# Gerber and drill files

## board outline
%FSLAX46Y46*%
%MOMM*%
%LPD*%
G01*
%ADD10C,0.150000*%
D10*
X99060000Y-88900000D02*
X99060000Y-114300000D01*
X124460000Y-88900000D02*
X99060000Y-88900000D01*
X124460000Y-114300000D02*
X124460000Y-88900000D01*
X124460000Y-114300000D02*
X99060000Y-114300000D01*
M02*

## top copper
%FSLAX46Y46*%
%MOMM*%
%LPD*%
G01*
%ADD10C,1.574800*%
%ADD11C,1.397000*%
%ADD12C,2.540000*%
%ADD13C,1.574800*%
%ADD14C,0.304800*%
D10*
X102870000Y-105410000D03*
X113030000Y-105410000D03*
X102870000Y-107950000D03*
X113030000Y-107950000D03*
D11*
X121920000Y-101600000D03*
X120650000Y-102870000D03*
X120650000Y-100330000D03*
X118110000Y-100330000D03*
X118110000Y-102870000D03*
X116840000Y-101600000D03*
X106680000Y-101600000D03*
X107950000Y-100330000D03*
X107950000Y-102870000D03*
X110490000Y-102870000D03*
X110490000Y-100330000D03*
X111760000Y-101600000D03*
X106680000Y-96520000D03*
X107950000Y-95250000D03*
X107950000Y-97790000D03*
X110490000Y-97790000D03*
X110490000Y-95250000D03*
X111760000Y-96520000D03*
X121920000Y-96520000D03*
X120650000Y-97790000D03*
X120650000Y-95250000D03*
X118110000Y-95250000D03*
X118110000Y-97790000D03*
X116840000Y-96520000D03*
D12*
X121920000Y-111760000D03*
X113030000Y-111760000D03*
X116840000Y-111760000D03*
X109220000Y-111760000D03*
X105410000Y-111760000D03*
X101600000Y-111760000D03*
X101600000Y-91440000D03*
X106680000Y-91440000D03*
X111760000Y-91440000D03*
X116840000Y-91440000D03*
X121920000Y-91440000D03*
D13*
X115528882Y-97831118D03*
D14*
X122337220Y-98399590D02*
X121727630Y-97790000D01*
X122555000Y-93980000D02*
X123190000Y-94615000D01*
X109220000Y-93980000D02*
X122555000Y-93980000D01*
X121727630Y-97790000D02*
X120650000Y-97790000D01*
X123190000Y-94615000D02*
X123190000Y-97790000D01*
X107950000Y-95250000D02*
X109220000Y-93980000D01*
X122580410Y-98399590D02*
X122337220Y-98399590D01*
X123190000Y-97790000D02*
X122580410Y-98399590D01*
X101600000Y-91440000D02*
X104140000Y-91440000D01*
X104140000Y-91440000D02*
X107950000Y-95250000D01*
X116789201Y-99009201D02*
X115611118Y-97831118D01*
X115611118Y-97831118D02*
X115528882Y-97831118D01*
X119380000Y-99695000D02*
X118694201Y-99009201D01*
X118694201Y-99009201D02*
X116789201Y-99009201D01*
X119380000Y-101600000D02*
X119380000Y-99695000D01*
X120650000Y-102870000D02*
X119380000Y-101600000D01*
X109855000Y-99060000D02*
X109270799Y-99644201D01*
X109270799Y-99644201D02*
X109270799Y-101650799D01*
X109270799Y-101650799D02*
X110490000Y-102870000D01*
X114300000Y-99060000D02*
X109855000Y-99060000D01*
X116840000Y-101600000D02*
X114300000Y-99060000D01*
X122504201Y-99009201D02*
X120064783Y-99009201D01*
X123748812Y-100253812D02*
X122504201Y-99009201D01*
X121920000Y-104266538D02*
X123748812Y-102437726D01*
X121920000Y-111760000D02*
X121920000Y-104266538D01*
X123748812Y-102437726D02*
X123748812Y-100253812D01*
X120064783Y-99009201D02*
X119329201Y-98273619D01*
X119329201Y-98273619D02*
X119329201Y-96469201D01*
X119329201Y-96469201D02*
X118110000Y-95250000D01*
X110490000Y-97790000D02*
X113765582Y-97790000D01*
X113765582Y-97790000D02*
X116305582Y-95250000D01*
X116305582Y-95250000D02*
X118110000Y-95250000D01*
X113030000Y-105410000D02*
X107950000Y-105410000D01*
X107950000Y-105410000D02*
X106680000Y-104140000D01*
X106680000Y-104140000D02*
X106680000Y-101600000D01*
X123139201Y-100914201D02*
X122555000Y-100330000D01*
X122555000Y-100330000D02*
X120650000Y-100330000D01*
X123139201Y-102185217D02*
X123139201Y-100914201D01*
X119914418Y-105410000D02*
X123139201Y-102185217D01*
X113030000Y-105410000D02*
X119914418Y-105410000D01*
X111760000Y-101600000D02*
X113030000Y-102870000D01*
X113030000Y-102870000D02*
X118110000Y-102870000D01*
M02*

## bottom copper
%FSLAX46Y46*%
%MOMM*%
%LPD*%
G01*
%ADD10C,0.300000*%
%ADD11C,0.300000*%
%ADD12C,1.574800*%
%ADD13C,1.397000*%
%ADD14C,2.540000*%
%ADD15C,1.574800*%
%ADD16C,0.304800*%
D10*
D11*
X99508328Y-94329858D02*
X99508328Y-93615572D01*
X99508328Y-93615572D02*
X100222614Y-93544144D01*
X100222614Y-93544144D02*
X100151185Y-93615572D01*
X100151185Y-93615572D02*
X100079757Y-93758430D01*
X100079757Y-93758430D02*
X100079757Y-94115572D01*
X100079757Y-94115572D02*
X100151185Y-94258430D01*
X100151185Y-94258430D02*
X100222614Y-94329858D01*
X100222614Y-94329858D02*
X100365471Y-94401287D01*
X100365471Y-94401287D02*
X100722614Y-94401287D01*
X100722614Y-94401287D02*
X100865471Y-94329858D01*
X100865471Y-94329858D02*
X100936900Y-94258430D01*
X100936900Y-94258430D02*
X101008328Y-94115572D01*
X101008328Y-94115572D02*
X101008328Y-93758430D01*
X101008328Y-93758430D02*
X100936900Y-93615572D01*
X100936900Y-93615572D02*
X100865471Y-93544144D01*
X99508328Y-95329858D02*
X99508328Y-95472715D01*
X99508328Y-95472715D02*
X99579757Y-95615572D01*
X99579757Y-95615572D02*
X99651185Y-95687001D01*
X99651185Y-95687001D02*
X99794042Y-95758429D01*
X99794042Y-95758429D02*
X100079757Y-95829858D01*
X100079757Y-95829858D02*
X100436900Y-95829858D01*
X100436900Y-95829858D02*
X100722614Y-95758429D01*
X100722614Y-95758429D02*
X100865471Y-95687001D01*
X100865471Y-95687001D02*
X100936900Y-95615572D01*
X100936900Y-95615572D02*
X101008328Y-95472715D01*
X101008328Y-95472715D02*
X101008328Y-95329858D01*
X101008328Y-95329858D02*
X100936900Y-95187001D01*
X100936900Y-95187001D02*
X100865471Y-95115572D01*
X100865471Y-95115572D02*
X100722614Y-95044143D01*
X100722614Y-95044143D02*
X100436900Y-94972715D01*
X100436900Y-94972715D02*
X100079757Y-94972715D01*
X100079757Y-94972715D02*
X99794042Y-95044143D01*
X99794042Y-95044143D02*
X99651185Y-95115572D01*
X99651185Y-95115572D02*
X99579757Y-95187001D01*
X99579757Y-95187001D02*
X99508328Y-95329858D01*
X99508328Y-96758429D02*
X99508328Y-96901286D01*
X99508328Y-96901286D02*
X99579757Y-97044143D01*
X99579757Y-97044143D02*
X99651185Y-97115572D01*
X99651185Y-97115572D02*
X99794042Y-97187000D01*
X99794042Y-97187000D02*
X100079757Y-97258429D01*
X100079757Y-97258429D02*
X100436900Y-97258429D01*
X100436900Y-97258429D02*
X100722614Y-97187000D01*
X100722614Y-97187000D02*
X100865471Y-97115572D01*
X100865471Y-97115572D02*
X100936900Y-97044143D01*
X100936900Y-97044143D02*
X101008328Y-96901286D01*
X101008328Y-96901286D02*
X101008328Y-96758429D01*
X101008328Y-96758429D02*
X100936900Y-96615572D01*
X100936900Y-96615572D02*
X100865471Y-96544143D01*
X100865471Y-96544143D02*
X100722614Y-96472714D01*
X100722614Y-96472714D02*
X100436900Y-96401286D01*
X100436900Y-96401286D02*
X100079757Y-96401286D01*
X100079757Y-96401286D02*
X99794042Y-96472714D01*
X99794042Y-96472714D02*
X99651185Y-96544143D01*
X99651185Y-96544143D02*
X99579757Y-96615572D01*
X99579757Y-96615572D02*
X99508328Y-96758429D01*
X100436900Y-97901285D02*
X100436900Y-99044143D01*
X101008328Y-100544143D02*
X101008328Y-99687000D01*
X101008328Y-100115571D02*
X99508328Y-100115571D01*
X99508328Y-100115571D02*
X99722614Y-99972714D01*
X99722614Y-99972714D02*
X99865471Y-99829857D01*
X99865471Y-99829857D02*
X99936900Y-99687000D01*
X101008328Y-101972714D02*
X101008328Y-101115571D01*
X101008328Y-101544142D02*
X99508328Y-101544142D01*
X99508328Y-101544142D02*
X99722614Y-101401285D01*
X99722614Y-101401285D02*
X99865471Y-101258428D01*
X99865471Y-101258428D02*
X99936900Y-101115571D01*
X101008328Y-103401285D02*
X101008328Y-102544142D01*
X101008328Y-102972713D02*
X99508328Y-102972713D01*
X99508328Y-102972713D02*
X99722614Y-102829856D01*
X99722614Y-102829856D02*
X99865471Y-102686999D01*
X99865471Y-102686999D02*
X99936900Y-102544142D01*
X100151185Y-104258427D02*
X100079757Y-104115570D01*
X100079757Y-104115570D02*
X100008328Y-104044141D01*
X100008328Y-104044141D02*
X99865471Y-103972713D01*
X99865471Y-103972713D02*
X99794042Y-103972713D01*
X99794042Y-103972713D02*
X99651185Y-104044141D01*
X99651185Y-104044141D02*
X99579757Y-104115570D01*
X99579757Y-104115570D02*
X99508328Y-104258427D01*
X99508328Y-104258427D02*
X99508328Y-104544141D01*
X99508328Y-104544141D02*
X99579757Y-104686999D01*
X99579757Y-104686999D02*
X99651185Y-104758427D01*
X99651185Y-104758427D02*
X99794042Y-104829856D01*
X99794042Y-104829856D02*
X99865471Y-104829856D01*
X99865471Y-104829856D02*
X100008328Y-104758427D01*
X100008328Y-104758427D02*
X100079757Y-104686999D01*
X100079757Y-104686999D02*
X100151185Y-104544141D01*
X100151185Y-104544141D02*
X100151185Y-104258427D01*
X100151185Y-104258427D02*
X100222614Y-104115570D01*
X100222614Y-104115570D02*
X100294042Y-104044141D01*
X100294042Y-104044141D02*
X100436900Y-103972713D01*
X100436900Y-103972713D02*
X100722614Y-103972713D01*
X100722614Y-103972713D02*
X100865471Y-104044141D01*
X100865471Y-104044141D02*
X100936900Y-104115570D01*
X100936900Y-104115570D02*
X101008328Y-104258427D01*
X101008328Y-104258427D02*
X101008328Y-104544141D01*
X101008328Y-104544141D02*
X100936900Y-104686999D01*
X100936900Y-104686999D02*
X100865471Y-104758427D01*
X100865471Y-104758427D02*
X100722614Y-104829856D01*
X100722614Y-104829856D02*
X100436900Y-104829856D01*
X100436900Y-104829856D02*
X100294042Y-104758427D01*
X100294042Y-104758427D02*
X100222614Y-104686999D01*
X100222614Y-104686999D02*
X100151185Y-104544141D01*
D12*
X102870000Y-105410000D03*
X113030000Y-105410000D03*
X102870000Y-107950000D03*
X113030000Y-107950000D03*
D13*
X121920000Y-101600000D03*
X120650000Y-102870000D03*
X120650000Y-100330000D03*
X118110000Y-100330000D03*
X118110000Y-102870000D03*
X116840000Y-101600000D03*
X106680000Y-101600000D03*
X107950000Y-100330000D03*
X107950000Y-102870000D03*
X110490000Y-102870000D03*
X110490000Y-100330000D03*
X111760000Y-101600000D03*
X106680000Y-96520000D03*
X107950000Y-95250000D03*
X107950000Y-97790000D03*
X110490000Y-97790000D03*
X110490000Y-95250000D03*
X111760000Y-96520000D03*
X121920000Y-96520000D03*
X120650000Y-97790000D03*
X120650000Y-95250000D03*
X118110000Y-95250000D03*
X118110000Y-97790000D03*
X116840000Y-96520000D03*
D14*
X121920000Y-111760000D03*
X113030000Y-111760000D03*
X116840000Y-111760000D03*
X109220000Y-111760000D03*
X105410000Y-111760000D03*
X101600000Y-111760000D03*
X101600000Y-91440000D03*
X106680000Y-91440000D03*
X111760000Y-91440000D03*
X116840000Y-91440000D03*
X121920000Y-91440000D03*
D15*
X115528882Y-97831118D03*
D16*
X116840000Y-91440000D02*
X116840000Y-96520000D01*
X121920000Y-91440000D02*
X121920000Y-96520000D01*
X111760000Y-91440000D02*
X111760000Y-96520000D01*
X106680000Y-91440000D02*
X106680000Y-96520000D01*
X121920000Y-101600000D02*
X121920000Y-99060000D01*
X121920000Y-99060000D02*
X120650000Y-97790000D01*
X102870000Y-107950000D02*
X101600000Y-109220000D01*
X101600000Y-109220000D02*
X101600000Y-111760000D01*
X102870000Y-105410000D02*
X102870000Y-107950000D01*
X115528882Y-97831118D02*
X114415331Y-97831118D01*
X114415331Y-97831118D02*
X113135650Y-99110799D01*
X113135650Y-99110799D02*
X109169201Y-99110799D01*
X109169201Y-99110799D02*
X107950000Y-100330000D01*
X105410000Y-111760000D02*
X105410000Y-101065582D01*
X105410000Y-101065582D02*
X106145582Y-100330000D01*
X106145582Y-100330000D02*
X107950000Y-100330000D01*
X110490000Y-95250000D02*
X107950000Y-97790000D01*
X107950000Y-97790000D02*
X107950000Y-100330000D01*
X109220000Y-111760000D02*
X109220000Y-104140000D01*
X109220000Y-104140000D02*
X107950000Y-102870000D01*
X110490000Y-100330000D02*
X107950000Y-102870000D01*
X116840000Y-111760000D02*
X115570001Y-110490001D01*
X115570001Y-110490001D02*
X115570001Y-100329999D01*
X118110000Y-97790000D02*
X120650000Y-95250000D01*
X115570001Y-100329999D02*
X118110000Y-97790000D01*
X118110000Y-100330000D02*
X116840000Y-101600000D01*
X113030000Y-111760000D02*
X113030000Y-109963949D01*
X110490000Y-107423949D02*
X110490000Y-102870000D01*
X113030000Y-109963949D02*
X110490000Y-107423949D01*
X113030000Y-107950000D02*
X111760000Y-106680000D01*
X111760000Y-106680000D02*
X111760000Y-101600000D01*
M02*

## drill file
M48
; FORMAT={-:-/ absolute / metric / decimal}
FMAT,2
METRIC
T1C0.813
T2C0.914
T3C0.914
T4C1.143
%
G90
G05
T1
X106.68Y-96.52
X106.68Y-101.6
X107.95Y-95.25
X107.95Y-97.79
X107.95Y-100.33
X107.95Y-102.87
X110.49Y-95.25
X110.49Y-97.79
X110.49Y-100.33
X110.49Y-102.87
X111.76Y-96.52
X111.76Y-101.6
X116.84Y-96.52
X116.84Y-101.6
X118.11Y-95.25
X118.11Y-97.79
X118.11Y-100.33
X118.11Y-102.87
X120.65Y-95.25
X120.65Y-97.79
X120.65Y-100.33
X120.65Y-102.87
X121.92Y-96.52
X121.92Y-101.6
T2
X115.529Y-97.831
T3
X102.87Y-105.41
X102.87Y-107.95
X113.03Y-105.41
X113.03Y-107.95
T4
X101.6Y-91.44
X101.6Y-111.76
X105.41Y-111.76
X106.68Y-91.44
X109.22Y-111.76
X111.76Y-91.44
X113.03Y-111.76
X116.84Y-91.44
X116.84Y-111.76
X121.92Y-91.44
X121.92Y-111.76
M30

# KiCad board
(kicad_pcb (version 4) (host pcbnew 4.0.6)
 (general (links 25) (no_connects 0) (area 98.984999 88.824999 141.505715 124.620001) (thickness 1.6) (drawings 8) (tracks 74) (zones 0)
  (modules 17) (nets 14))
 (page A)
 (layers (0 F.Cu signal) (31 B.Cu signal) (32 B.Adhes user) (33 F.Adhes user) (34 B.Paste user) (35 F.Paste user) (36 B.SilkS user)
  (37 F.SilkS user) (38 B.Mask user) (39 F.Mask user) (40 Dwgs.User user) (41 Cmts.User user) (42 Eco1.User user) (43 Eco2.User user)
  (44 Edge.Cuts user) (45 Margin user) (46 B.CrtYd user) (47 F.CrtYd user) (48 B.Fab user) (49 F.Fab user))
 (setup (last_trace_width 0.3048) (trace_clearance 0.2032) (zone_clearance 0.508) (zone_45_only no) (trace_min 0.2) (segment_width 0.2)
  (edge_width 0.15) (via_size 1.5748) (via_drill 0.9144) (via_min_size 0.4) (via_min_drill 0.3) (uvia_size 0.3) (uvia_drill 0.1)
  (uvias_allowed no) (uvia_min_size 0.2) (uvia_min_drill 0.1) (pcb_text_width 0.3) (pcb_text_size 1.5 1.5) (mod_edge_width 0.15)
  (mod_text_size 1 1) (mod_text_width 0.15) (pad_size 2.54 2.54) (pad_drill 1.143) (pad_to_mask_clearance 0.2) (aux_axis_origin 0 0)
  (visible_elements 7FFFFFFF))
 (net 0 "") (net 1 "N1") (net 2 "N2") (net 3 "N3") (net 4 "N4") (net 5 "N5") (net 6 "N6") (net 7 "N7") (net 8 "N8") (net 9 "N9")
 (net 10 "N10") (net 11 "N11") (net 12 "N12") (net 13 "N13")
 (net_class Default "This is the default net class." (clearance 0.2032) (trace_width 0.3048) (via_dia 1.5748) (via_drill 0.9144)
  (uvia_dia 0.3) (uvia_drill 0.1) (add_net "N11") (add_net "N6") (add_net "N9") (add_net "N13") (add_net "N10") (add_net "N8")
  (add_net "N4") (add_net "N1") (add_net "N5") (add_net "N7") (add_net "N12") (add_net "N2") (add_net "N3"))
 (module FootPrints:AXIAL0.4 (layer F.Cu) (at 107.95 105.41)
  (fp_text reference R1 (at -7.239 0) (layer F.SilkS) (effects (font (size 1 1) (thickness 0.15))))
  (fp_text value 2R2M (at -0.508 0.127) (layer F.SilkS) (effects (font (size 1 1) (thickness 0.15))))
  (pad 1 thru_hole circle (at -5.08 0) (size 1.5748 1.5748) (drill 0.9144) (layers *.Cu *.Mask F.SilkS) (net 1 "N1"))
  (pad 2 thru_hole circle (at 5.08 0) (size 1.5748 1.5748) (drill 0.9144) (layers *.Cu *.Mask F.SilkS) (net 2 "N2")))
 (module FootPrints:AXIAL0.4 (layer F.Cu) (at 107.95 107.95)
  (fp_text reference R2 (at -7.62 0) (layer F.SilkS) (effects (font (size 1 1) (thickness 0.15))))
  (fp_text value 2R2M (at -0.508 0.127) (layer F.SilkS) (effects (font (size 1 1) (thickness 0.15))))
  (pad 1 thru_hole circle (at -5.08 0) (size 1.5748 1.5748) (drill 0.9144) (layers *.Cu *.Mask F.SilkS) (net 1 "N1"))
  (pad 2 thru_hole circle (at 5.08 0) (size 1.5748 1.5748) (drill 0.9144) (layers *.Cu *.Mask F.SilkS) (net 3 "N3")))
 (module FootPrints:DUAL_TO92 (layer F.Cu) (at 119.38 101.6 90)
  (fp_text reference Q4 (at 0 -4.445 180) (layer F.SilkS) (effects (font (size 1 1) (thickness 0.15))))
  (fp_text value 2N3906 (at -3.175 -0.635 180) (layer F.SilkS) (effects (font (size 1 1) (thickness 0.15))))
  (pad 2 thru_hole circle (at 0 2.54 90) (size 1.397 1.397) (drill 0.8128) (layers *.Cu *.Mask F.SilkS) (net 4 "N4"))
  (pad 3 thru_hole circle (at -1.27 1.27 90) (size 1.397 1.397) (drill 0.8128) (layers *.Cu *.Mask F.SilkS) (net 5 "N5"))
  (pad 1 thru_hole circle (at 1.27 1.27 90) (size 1.397 1.397) (drill 0.8128) (layers *.Cu *.Mask F.SilkS) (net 2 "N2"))
  (pad 6 thru_hole circle (at 1.27 -1.27 90) (size 1.397 1.397) (drill 0.8128) (layers *.Cu *.Mask F.SilkS) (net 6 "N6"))
  (pad 4 thru_hole circle (at -1.27 -1.27 90) (size 1.397 1.397) (drill 0.8128) (layers *.Cu *.Mask F.SilkS) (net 3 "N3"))
  (pad 5 thru_hole circle (at 0 -2.54 90) (size 1.397 1.397) (drill 0.8128) (layers *.Cu *.Mask F.SilkS) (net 6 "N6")))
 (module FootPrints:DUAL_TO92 (layer F.Cu) (at 109.22 101.6 270)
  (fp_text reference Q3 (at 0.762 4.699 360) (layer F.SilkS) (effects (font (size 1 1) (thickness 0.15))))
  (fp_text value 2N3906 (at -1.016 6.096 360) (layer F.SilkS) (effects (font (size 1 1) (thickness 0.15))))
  (pad 2 thru_hole circle (at 0 2.54 270) (size 1.397 1.397) (drill 0.8128) (layers *.Cu *.Mask F.SilkS) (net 2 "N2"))
  (pad 3 thru_hole circle (at -1.27 1.27 270) (size 1.397 1.397) (drill 0.8128) (layers *.Cu *.Mask F.SilkS) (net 5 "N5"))
  (pad 1 thru_hole circle (at 1.27 1.27 270) (size 1.397 1.397) (drill 0.8128) (layers *.Cu *.Mask F.SilkS) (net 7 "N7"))
  (pad 6 thru_hole circle (at 1.27 -1.27 270) (size 1.397 1.397) (drill 0.8128) (layers *.Cu *.Mask F.SilkS) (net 6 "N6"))
  (pad 4 thru_hole circle (at -1.27 -1.27 270) (size 1.397 1.397) (drill 0.8128) (layers *.Cu *.Mask F.SilkS) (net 7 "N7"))
  (pad 5 thru_hole circle (at 0 -2.54 270) (size 1.397 1.397) (drill 0.8128) (layers *.Cu *.Mask F.SilkS) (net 3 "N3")))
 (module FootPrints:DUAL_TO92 (layer F.Cu) (at 109.22 96.52 270)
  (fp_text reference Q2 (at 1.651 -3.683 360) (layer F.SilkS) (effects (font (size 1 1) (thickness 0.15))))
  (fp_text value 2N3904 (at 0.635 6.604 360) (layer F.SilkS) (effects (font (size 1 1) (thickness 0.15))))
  (pad 2 thru_hole circle (at 0 2.54 270) (size 1.397 1.397) (drill 0.8128) (layers *.Cu *.Mask F.SilkS) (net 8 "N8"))
  (pad 3 thru_hole circle (at -1.27 1.27 270) (size 1.397 1.397) (drill 0.8128) (layers *.Cu *.Mask F.SilkS) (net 4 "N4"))
  (pad 1 thru_hole circle (at 1.27 1.27 270) (size 1.397 1.397) (drill 0.8128) (layers *.Cu *.Mask F.SilkS) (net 5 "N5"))
  (pad 6 thru_hole circle (at 1.27 -1.27 270) (size 1.397 1.397) (drill 0.8128) (layers *.Cu *.Mask F.SilkS) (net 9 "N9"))
  (pad 4 thru_hole circle (at -1.27 -1.27 270) (size 1.397 1.397) (drill 0.8128) (layers *.Cu *.Mask F.SilkS) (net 5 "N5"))
  (pad 5 thru_hole circle (at 0 -2.54 270) (size 1.397 1.397) (drill 0.8128) (layers *.Cu *.Mask F.SilkS) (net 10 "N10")))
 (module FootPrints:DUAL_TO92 (layer F.Cu) (at 119.38 96.52 90)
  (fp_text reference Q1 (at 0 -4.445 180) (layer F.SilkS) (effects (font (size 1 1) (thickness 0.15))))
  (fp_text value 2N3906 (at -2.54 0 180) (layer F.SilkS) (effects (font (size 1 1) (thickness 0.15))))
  (pad 2 thru_hole circle (at 0 2.54 90) (size 1.397 1.397) (drill 0.8128) (layers *.Cu *.Mask F.SilkS) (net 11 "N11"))
  (pad 3 thru_hole circle (at -1.27 1.27 90) (size 1.397 1.397) (drill 0.8128) (layers *.Cu *.Mask F.SilkS) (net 4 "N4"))
  (pad 1 thru_hole circle (at 1.27 1.27 90) (size 1.397 1.397) (drill 0.8128) (layers *.Cu *.Mask F.SilkS) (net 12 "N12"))
  (pad 6 thru_hole circle (at 1.27 -1.27 90) (size 1.397 1.397) (drill 0.8128) (layers *.Cu *.Mask F.SilkS) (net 9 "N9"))
  (pad 4 thru_hole circle (at -1.27 -1.27 90) (size 1.397 1.397) (drill 0.8128) (layers *.Cu *.Mask F.SilkS) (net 12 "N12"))
  (pad 5 thru_hole circle (at 0 -2.54 90) (size 1.397 1.397) (drill 0.8128) (layers *.Cu *.Mask F.SilkS) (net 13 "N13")))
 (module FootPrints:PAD (layer F.Cu) (at 121.92 114.3)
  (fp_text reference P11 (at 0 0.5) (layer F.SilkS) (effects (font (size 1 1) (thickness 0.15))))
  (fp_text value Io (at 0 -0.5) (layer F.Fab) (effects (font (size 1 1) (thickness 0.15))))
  (pad 1 thru_hole circle (at 0 -2.54) (size 2.54 2.54) (drill 1.143) (layers *.Cu *.Mask F.SilkS) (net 9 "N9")))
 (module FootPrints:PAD (layer F.Cu) (at 113.03 114.3)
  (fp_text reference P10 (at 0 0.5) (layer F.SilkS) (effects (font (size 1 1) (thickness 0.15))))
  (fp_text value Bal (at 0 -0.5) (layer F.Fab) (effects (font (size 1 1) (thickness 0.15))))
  (pad 1 thru_hole circle (at 0 -2.54) (size 2.54 2.54) (drill 1.143) (layers *.Cu *.Mask F.SilkS) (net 6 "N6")))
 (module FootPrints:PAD (layer F.Cu) (at 116.84 114.3)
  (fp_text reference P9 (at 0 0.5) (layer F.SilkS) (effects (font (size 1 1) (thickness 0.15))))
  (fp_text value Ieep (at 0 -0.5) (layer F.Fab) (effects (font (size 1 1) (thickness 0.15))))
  (pad 1 thru_hole circle (at 0 -2.54) (size 2.54 2.54) (drill 1.143) (layers *.Cu *.Mask F.SilkS) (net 12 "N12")))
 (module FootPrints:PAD (layer F.Cu) (at 109.22 114.3)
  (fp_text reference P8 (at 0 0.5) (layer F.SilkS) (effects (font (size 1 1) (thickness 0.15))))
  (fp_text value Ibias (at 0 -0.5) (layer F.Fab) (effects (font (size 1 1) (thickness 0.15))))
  (pad 1 thru_hole circle (at 0 -2.54) (size 2.54 2.54) (drill 1.143) (layers *.Cu *.Mask F.SilkS) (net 7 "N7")))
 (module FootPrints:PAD (layer F.Cu) (at 105.41 114.3)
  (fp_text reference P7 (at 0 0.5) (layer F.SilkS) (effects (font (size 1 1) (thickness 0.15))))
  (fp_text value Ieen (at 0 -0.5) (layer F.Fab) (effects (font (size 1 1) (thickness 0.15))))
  (pad 1 thru_hole circle (at 0 -2.54) (size 2.54 2.54) (drill 1.143) (layers *.Cu *.Mask F.SilkS) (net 5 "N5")))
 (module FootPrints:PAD (layer F.Cu) (at 101.6 114.3)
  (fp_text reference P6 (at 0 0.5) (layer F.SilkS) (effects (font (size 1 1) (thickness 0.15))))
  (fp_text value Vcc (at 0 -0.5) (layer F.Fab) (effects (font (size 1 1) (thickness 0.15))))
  (pad 1 thru_hole circle (at 0 -2.54) (size 2.54 2.54) (drill 1.143) (layers *.Cu *.Mask F.SilkS) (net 1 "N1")))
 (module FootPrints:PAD (layer F.Cu) (at 101.6 93.98)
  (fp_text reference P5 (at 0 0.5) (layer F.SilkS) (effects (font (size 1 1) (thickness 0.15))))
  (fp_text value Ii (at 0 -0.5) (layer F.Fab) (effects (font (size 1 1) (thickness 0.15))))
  (pad 1 thru_hole circle (at 0 -2.54) (size 2.54 2.54) (drill 1.143) (layers *.Cu *.Mask F.SilkS) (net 4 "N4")))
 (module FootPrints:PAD (layer F.Cu) (at 106.68 93.98)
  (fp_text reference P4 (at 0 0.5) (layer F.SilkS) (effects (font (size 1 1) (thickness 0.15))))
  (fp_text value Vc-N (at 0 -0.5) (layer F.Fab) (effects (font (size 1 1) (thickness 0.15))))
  (pad 1 thru_hole circle (at 0 -2.54) (size 2.54 2.54) (drill 1.143) (layers *.Cu *.Mask F.SilkS) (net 8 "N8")))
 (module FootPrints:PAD (layer F.Cu) (at 111.76 93.98)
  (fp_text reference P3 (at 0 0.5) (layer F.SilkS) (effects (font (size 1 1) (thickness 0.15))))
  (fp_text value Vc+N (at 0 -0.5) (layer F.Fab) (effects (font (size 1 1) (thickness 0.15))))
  (pad 1 thru_hole circle (at 0 -2.54) (size 2.54 2.54) (drill 1.143) (layers *.Cu *.Mask F.SilkS) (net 10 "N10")))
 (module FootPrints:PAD (layer F.Cu) (at 116.84 93.98)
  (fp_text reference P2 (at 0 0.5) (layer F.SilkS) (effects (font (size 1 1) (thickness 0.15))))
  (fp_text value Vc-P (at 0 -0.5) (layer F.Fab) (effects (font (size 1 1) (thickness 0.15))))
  (pad 1 thru_hole circle (at 0 -2.54) (size 2.54 2.54) (drill 1.143) (layers *.Cu *.Mask F.SilkS)))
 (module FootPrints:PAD (layer F.Cu) (at 121.92 93.98)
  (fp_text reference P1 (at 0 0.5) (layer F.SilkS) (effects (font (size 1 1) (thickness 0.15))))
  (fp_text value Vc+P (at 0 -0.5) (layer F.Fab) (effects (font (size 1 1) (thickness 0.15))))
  (pad 1 thru_hole circle (at 0 -2.54) (size 2.54 2.54) (drill 1.143) (layers *.Cu *.Mask F.SilkS) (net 11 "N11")))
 (gr_line (start 99.06 88.9) (end 99.06 114.3) (angle 90) (layer Edge.Cuts) (width 0.15))
 (gr_line (start 124.46 88.9) (end 99.06 88.9) (angle 90) (layer Edge.Cuts) (width 0.15))
 (gr_line (start 124.46 114.3) (end 124.46 88.9) (angle 90) (layer Edge.Cuts) (width 0.15))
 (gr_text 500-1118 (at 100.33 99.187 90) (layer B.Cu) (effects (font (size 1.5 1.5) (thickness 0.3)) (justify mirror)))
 (gr_line (start 124.46 114.3) (end 99.06 114.3) (angle 90) (layer Edge.Cuts) (width 0.15))
 (segment (start 116.84 91.44) (end 116.84 96.52) (width 0.3048) (layer B.Cu) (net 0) (status 30))
 (segment (start 121.92 91.44) (end 121.92 96.52) (width 0.3048) (layer B.Cu) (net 11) (status 30))
 (segment (start 111.76 91.44) (end 111.76 96.52) (width 0.3048) (layer B.Cu) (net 10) (status 30))
 (segment (start 106.68 91.44) (end 106.68 96.52) (width 0.3048) (layer B.Cu) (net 8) (status 30))
 (segment (start 122.33722 98.39959) (end 121.72763 97.79) (width 0.3048) (layer F.Cu) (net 4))
 (segment (start 122.555 93.98) (end 123.19 94.615) (width 0.3048) (layer F.Cu) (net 4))
 (segment (start 109.22 93.98) (end 122.555 93.98) (width 0.3048) (layer F.Cu) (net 4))
 (segment (start 121.72763 97.79) (end 120.65 97.79) (width 0.3048) (layer F.Cu) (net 4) (status 20))
 (segment (start 123.19 94.615) (end 123.19 97.79) (width 0.3048) (layer F.Cu) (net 4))
 (segment (start 107.95 95.25) (end 109.22 93.98) (width 0.3048) (layer F.Cu) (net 4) (status 10))
 (segment (start 122.58041 98.39959) (end 122.33722 98.39959) (width 0.3048) (layer F.Cu) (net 4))
 (segment (start 123.19 97.79) (end 122.58041 98.39959) (width 0.3048) (layer F.Cu) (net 4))
 (segment (start 101.6 91.44) (end 104.14 91.44) (width 0.3048) (layer F.Cu) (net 4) (status 10))
 (segment (start 104.14 91.44) (end 107.95 95.25) (width 0.3048) (layer F.Cu) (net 4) (status 20))
 (segment (start 121.92 101.6) (end 121.92 99.06) (width 0.3048) (layer B.Cu) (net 4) (status 10))
 (segment (start 121.92 99.06) (end 120.65 97.79) (width 0.3048) (layer B.Cu) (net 4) (status 20))
 (segment (start 102.87 107.95) (end 101.6 109.22) (width 0.3048) (layer B.Cu) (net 1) (status 10))
 (segment (start 101.6 109.22) (end 101.6 111.76) (width 0.3048) (layer B.Cu) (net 1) (status 20))
 (segment (start 102.87 105.41) (end 102.87 107.95) (width 0.3048) (layer B.Cu) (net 1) (status 30))
 (segment (start 115.528882 97.831118) (end 114.415331 97.831118) (width 0.3048) (layer B.Cu) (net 5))
 (segment (start 114.415331 97.831118) (end 113.13565 99.110799) (width 0.3048) (layer B.Cu) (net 5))
 (segment (start 113.13565 99.110799) (end 109.169201 99.110799) (width 0.3048) (layer B.Cu) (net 5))
 (segment (start 109.169201 99.110799) (end 107.95 100.33) (width 0.3048) (layer B.Cu) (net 5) (status 20))
 (segment (start 116.789201 99.009201) (end 115.611118 97.831118) (width 0.3048) (layer F.Cu) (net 5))
 (segment (start 115.611118 97.831118) (end 115.528882 97.831118) (width 0.3048) (layer F.Cu) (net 5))
 (via (at 115.528882 97.831118) (size 1.5748) (drill 0.9144) (layers F.Cu B.Cu) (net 5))
 (segment (start 119.38 99.695) (end 118.694201 99.009201) (width 0.3048) (layer F.Cu) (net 5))
 (segment (start 118.694201 99.009201) (end 116.789201 99.009201) (width 0.3048) (layer F.Cu) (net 5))
 (segment (start 119.38 101.6) (end 119.38 99.695) (width 0.3048) (layer F.Cu) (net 5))
 (segment (start 120.65 102.87) (end 119.38 101.6) (width 0.3048) (layer F.Cu) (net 5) (status 10))
 (segment (start 105.41 111.76) (end 105.41 101.065582) (width 0.3048) (layer B.Cu) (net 5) (status 10))
 (segment (start 105.41 101.065582) (end 106.145582 100.33) (width 0.3048) (layer B.Cu) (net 5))
 (segment (start 106.145582 100.33) (end 107.95 100.33) (width 0.3048) (layer B.Cu) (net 5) (status 20))
 (segment (start 110.49 95.25) (end 107.95 97.79) (width 0.3048) (layer B.Cu) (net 5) (status 30))
 (segment (start 107.95 97.79) (end 107.95 100.33) (width 0.3048) (layer B.Cu) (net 5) (status 30))
 (segment (start 109.22 111.76) (end 109.22 104.14) (width 0.3048) (layer B.Cu) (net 7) (status 10))
 (segment (start 109.22 104.14) (end 107.95 102.87) (width 0.3048) (layer B.Cu) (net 7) (status 20))
 (segment (start 110.49 100.33) (end 107.95 102.87) (width 0.3048) (layer B.Cu) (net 7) (status 30))
 (segment (start 116.84 111.76) (end 115.570001 110.490001) (width 0.3048) (layer B.Cu) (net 12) (status 10))
 (segment (start 115.570001 110.490001) (end 115.570001 100.329999) (width 0.3048) (layer B.Cu) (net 12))
 (segment (start 118.11 97.79) (end 120.65 95.25) (width 0.3048) (layer B.Cu) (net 12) (status 30))
 (segment (start 115.570001 100.329999) (end 118.11 97.79) (width 0.3048) (layer B.Cu) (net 12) (status 20))
 (segment (start 118.11 100.33) (end 116.84 101.6) (width 0.3048) (layer B.Cu) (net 6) (status 30))
 (segment (start 109.855 99.06) (end 109.270799 99.644201) (width 0.3048) (layer F.Cu) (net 6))
 (segment (start 109.270799 99.644201) (end 109.270799 101.650799) (width 0.3048) (layer F.Cu) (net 6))
 (segment (start 109.270799 101.650799) (end 110.49 102.87) (width 0.3048) (layer F.Cu) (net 6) (status 20))
 (segment (start 114.3 99.06) (end 109.855 99.06) (width 0.3048) (layer F.Cu) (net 6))
 (segment (start 116.84 101.6) (end 114.3 99.06) (width 0.3048) (layer F.Cu) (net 6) (status 10))
 (segment (start 113.03 111.76) (end 113.03 109.963949) (width 0.3048) (layer B.Cu) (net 6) (status 10))
 (segment (start 110.49 107.423949) (end 110.49 102.87) (width 0.3048) (layer B.Cu) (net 6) (status 20))
 (segment (start 113.03 109.963949) (end 110.49 107.423949) (width 0.3048) (layer B.Cu) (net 6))
 (segment (start 122.504201 99.009201) (end 120.064783 99.009201) (width 0.3048) (layer F.Cu) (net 9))
 (segment (start 123.748812 100.253812) (end 122.504201 99.009201) (width 0.3048) (layer F.Cu) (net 9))
 (segment (start 121.92 104.266538) (end 123.748812 102.437726) (width 0.3048) (layer F.Cu) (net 9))
 (segment (start 121.92 111.76) (end 121.92 104.266538) (width 0.3048) (layer F.Cu) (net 9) (status 10))
 (segment (start 123.748812 102.437726) (end 123.748812 100.253812) (width 0.3048) (layer F.Cu) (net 9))
 (segment (start 120.064783 99.009201) (end 119.329201 98.273619) (width 0.3048) (layer F.Cu) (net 9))
 (segment (start 119.329201 98.273619) (end 119.329201 96.469201) (width 0.3048) (layer F.Cu) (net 9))
 (segment (start 119.329201 96.469201) (end 118.11 95.25) (width 0.3048) (layer F.Cu) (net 9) (status 20))
 (segment (start 110.49 97.79) (end 113.765582 97.79) (width 0.3048) (layer F.Cu) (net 9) (status 10))
 (segment (start 113.765582 97.79) (end 116.305582 95.25) (width 0.3048) (layer F.Cu) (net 9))
 (segment (start 116.305582 95.25) (end 118.11 95.25) (width 0.3048) (layer F.Cu) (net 9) (status 20))
 (segment (start 113.03 105.41) (end 107.95 105.41) (width 0.3048) (layer F.Cu) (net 2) (status 10))
 (segment (start 107.95 105.41) (end 106.68 104.14) (width 0.3048) (layer F.Cu) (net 2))
 (segment (start 106.68 104.14) (end 106.68 101.6) (width 0.3048) (layer F.Cu) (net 2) (status 20))
 (segment (start 123.139201 100.914201) (end 122.555 100.33) (width 0.3048) (layer F.Cu) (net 2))
 (segment (start 122.555 100.33) (end 120.65 100.33) (width 0.3048) (layer F.Cu) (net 2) (status 20))
 (segment (start 123.139201 102.185217) (end 123.139201 100.914201) (width 0.3048) (layer F.Cu) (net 2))
 (segment (start 119.914418 105.41) (end 123.139201 102.185217) (width 0.3048) (layer F.Cu) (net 2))
 (segment (start 113.03 105.41) (end 119.914418 105.41) (width 0.3048) (layer F.Cu) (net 2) (status 10))
 (segment (start 111.76 101.6) (end 113.03 102.87) (width 0.3048) (layer F.Cu) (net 3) (status 10))
 (segment (start 113.03 102.87) (end 118.11 102.87) (width 0.3048) (layer F.Cu) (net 3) (status 20))
 (segment (start 113.03 107.95) (end 111.76 106.68) (width 0.3048) (layer B.Cu) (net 3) (status 10))
 (segment (start 111.76 106.68) (end 111.76 101.6) (width 0.3048) (layer B.Cu) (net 3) (status 20)))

